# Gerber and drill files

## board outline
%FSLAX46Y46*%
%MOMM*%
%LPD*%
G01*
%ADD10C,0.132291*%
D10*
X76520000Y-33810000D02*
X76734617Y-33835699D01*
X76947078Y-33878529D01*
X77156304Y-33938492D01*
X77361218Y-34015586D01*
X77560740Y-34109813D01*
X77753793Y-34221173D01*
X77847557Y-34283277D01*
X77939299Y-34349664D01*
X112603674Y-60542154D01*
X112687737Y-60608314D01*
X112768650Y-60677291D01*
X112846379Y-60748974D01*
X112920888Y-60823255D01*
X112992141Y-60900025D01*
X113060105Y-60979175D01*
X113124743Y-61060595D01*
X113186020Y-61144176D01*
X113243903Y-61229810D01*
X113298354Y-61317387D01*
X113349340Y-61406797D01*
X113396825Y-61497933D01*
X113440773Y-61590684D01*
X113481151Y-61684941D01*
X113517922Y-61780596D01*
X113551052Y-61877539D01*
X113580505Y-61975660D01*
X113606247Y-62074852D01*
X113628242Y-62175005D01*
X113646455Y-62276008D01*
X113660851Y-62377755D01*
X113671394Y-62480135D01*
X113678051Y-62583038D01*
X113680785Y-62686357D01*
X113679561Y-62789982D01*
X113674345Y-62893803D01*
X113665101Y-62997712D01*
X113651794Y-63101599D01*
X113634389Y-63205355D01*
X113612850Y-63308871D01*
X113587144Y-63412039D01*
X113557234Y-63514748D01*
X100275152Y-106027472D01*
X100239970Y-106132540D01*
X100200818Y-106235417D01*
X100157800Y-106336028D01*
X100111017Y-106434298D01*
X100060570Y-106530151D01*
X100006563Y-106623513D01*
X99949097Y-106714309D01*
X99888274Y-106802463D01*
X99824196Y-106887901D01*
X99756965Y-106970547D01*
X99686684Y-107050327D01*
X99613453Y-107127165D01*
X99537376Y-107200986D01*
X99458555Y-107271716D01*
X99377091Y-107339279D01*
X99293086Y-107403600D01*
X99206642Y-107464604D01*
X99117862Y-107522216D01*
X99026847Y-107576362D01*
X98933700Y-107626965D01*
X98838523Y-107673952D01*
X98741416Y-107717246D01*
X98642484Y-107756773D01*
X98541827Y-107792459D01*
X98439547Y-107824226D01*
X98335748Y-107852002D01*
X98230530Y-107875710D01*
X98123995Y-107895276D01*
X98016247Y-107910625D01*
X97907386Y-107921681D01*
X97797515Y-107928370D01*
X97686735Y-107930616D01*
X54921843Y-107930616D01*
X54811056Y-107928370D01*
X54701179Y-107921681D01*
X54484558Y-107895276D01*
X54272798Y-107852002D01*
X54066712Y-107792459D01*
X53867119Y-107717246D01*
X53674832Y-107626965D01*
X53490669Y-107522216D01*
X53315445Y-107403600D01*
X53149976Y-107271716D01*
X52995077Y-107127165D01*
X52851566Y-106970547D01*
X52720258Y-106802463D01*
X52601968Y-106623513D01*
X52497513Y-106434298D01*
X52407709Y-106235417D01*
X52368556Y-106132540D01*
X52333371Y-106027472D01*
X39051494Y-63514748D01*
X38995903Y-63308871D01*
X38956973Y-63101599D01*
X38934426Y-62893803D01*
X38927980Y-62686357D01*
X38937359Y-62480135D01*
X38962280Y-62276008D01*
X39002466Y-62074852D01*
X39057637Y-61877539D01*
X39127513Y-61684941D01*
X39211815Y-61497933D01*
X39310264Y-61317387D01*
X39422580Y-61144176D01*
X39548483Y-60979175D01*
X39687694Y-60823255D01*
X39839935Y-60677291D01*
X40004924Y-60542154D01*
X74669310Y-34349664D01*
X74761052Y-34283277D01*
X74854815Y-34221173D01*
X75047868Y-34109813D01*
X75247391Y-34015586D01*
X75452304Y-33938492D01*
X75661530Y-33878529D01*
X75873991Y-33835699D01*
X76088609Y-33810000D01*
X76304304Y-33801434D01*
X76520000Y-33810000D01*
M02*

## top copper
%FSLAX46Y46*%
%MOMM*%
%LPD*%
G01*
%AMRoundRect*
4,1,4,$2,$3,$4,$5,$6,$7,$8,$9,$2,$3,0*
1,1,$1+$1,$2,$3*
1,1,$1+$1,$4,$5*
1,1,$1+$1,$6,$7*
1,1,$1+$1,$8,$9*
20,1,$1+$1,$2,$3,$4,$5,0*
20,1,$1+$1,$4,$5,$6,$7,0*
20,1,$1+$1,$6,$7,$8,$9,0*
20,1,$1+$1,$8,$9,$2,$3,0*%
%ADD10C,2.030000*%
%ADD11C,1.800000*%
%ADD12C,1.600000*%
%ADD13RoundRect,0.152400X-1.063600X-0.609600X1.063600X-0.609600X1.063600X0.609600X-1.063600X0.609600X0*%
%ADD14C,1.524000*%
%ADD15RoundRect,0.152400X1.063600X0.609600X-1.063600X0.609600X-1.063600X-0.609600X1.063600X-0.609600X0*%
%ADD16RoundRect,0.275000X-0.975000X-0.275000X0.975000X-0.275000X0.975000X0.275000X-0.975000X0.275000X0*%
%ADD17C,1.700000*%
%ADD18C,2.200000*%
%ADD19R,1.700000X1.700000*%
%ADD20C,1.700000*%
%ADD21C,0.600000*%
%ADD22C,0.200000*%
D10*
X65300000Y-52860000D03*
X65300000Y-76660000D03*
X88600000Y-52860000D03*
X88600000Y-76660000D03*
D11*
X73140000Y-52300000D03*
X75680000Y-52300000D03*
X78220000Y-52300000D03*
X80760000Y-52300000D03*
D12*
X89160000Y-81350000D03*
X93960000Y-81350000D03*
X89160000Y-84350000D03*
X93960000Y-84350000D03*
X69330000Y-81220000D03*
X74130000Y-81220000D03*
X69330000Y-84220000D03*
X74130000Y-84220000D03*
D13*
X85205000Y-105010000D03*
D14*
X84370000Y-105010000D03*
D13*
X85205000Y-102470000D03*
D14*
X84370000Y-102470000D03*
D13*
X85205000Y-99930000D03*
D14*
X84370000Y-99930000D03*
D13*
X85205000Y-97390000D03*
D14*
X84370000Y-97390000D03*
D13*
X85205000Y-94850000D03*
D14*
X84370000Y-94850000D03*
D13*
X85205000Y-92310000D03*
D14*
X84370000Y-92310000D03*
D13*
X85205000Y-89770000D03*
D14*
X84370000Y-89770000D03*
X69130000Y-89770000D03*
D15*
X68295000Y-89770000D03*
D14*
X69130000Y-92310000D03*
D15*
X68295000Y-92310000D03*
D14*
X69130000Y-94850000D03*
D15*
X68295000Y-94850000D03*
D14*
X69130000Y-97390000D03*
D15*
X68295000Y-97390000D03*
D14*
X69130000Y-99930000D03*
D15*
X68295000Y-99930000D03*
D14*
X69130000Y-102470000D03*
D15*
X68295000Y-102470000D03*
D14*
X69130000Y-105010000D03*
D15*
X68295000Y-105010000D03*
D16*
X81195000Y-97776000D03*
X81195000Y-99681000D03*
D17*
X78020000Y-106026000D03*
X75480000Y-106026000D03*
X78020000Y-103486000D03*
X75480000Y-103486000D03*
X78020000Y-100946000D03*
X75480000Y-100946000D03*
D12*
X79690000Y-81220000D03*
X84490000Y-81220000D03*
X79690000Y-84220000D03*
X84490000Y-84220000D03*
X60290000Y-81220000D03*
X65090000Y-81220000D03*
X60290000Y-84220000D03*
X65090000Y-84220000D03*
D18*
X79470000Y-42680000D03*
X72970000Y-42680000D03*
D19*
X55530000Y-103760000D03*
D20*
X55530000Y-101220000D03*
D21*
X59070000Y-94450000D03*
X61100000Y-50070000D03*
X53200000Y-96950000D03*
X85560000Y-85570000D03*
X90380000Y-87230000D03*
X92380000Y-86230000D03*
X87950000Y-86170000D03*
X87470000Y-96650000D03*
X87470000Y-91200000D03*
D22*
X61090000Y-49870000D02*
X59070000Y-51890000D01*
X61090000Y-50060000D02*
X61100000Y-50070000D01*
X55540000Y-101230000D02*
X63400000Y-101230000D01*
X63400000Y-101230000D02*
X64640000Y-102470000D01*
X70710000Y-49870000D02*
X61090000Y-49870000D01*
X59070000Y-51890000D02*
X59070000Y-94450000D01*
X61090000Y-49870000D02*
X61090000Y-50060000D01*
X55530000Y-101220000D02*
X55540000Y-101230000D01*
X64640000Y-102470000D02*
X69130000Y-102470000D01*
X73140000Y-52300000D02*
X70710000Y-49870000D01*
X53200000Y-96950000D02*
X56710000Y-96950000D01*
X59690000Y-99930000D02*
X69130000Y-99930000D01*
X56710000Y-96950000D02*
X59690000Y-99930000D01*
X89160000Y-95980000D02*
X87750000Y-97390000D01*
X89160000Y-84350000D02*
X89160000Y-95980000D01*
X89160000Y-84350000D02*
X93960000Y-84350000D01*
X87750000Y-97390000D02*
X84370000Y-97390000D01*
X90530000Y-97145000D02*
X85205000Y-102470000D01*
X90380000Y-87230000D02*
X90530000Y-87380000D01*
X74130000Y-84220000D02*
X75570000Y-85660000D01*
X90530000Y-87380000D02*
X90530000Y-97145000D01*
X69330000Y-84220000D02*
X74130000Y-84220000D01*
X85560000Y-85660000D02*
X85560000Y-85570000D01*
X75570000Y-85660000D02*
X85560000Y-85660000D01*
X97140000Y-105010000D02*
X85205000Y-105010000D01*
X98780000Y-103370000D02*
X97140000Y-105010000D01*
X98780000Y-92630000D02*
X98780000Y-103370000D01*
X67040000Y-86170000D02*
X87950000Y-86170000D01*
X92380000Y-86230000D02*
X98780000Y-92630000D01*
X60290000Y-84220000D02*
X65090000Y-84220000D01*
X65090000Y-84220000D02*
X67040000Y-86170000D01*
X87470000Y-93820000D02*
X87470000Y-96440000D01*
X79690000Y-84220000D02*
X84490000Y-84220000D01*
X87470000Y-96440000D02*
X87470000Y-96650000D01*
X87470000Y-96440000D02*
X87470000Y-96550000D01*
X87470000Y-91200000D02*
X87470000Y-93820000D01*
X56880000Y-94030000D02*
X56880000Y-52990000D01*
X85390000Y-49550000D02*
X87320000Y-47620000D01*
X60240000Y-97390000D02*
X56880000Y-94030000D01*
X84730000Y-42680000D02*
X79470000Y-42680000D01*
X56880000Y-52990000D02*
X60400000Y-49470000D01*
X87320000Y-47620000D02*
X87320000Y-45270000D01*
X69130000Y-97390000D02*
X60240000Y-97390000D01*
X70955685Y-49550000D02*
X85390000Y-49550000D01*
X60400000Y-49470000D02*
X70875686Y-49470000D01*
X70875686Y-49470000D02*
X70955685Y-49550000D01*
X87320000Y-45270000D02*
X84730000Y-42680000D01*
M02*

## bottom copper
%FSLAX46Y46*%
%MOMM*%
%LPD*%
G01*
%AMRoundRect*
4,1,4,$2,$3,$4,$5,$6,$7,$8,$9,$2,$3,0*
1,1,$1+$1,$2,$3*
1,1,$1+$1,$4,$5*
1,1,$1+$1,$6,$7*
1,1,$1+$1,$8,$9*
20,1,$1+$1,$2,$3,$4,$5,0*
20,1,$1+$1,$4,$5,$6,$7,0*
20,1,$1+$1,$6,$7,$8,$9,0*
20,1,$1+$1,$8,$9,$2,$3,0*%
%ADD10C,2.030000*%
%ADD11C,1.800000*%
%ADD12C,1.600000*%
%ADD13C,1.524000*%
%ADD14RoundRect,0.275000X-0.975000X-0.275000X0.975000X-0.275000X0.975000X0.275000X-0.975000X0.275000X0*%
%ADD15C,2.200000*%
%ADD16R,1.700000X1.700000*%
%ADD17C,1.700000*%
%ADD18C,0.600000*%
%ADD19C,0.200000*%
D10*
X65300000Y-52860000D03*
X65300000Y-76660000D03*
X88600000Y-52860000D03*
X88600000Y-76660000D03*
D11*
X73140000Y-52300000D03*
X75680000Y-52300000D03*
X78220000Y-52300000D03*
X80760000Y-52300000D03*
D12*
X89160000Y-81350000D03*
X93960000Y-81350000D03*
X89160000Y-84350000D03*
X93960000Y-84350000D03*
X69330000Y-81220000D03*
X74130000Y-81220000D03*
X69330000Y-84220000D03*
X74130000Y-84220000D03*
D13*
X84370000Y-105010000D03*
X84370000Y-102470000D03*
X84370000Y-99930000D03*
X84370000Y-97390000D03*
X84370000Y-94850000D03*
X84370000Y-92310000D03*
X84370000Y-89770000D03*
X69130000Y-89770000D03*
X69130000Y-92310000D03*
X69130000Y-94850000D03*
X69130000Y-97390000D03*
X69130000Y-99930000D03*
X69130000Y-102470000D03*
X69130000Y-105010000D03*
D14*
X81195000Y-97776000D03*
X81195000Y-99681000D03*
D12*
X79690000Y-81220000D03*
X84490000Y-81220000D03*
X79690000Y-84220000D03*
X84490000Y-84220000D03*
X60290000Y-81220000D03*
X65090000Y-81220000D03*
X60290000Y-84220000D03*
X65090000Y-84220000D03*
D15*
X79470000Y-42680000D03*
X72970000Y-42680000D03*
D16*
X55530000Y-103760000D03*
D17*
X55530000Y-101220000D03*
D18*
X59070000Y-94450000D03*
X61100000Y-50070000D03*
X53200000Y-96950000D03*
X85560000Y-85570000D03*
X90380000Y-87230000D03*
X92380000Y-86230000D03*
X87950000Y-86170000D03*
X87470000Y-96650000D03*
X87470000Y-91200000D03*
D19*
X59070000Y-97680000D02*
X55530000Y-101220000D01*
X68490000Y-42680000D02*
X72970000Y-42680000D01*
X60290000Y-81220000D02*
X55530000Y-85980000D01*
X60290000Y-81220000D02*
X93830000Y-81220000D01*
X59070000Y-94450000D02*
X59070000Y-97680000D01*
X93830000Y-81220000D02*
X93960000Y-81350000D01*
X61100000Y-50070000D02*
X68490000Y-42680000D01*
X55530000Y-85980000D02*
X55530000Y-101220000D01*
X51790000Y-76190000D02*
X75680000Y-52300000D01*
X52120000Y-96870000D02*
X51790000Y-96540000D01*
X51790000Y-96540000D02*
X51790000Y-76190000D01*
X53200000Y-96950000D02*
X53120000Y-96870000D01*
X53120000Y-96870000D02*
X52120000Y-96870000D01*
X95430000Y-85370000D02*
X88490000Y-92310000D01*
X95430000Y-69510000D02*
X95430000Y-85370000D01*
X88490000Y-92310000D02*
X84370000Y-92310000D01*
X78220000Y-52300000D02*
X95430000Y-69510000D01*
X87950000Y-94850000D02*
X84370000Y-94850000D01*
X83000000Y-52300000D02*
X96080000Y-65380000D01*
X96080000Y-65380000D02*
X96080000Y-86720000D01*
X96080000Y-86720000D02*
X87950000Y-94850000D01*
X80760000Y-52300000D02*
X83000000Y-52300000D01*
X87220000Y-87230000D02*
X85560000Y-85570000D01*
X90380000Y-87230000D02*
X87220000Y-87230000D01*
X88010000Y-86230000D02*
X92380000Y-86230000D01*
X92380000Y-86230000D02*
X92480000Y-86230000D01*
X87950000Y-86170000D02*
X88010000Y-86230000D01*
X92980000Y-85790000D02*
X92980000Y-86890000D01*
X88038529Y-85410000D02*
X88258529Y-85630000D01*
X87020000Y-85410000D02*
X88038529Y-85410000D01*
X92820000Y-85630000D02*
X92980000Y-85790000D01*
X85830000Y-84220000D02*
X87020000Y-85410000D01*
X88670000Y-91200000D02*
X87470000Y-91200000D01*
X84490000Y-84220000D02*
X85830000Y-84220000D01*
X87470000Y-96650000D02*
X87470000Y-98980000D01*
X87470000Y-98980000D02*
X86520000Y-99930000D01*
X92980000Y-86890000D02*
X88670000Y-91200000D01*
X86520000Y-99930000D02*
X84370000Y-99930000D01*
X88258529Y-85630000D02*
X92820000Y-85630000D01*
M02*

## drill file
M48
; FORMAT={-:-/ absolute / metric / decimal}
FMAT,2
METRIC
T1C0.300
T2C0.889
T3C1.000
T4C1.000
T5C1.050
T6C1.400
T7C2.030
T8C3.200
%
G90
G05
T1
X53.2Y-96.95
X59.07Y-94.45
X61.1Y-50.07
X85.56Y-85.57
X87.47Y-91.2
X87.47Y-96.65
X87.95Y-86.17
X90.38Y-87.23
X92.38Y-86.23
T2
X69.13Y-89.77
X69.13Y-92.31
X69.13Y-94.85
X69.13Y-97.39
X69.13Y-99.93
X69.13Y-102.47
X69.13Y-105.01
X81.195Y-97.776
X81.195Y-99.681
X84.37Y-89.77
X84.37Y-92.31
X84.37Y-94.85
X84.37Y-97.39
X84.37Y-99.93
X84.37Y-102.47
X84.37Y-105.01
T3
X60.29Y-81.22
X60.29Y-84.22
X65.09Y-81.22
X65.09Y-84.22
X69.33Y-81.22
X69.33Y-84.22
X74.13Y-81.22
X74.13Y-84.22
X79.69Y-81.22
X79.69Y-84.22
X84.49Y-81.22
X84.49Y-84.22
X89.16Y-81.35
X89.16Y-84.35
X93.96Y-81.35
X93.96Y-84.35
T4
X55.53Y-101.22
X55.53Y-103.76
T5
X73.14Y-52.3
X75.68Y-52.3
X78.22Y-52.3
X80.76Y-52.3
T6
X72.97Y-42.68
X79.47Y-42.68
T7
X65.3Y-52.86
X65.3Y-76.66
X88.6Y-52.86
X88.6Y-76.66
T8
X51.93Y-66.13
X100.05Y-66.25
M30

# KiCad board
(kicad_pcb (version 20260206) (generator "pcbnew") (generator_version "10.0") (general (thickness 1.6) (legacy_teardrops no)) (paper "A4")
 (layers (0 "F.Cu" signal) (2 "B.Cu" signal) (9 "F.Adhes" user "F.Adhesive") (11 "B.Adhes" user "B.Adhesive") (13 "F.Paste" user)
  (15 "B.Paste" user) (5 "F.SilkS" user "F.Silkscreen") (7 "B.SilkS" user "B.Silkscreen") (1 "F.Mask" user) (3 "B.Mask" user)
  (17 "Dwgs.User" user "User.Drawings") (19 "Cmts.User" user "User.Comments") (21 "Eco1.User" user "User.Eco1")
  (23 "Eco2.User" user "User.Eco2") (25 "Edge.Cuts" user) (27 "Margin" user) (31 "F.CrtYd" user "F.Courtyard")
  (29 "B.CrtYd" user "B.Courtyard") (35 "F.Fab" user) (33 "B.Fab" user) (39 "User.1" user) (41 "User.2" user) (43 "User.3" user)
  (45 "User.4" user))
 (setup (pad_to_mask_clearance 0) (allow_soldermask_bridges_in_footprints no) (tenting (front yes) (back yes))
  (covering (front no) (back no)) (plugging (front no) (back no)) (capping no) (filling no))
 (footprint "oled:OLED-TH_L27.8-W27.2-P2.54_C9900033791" (layer "F.Cu") (at 76.95 52.3)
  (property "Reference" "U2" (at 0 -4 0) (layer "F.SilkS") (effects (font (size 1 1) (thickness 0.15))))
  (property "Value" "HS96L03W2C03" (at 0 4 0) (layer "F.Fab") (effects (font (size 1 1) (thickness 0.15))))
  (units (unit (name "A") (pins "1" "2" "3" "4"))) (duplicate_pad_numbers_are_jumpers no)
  (pad "" thru_hole circle (at -11.65 0.56) (size 2.03 2.03) (drill 2.03) (layers "*.Cu" "*.Mask") (remove_unused_layers no))
  (pad "" thru_hole circle (at -11.65 24.36) (size 2.03 2.03) (drill 2.03) (layers "*.Cu" "*.Mask") (remove_unused_layers no))
  (pad "" thru_hole circle (at 11.65 0.56) (size 2.03 2.03) (drill 2.03) (layers "*.Cu" "*.Mask") (remove_unused_layers no))
  (pad "" thru_hole circle (at 11.65 24.36) (size 2.03 2.03) (drill 2.03) (layers "*.Cu" "*.Mask") (remove_unused_layers no))
  (pad "1" thru_hole circle (at -3.81 0) (size 1.8 1.8) (drill 1.049986) (layers "*.Cu" "*.Mask") (remove_unused_layers no) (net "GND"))
  (pad "2" thru_hole circle (at -1.27 0) (size 1.8 1.8) (drill 1.049986) (layers "*.Cu" "*.Mask") (remove_unused_layers no) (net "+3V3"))
  (pad "3" thru_hole circle (at 1.27 0) (size 1.8 1.8) (drill 1.049986) (layers "*.Cu" "*.Mask") (remove_unused_layers no)
   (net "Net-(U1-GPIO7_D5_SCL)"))
  (pad "4" thru_hole circle (at 3.81 0) (size 1.8 1.8) (drill 1.049986) (layers "*.Cu" "*.Mask") (remove_unused_layers no)
   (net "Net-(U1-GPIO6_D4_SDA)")))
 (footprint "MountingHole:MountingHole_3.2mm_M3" (layer "F.Cu") (at 100.05 66.25)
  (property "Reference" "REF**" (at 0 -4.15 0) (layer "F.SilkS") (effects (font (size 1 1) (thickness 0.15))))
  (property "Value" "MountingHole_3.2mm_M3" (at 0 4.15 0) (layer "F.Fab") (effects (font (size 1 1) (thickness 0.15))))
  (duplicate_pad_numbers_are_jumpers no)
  (pad "" np_thru_hole circle (at 0 0) (size 3.2 3.2) (drill 3.2) (layers "*.Cu" "*.Mask")))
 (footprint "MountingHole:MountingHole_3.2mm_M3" (layer "F.Cu") (at 51.93 66.13)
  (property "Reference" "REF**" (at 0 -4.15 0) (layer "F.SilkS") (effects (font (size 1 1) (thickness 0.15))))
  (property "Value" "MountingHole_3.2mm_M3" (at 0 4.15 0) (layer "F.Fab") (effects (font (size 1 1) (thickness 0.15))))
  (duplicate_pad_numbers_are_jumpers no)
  (pad "" np_thru_hole circle (at 0 0) (size 3.2 3.2) (drill 3.2) (layers "*.Cu" "*.Mask")))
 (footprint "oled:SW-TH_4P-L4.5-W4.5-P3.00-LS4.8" (layer "F.Cu") (at 91.56 82.85)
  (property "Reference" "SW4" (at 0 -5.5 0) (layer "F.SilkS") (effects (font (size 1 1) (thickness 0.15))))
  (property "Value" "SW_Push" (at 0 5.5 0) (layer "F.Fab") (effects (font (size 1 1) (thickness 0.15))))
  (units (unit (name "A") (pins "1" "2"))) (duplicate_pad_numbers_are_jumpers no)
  (pad "1" thru_hole circle (at -2.4 -1.5) (size 1.6 1.6) (drill 0.999998) (layers "*.Cu" "*.Mask") (remove_unused_layers no) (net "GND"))
  (pad "1" thru_hole circle (at 2.4 -1.5) (size 1.6 1.6) (drill 0.999998) (layers "*.Cu" "*.Mask") (remove_unused_layers no) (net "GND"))
  (pad "2" thru_hole circle (at -2.4 1.5) (size 1.6 1.6) (drill 0.999998) (layers "*.Cu" "*.Mask") (remove_unused_layers no)
   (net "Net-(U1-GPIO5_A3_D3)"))
  (pad "2" thru_hole circle (at 2.4 1.5) (size 1.6 1.6) (drill 0.999998) (layers "*.Cu" "*.Mask") (remove_unused_layers no)
   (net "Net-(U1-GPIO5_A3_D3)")))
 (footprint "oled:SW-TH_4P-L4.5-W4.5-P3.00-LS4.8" (layer "F.Cu") (at 71.73 82.72)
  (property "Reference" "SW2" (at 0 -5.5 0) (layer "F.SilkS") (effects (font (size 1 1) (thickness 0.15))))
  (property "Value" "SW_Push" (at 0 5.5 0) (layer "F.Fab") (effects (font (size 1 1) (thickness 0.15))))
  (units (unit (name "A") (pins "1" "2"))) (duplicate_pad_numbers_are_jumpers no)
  (pad "1" thru_hole circle (at -2.4 -1.5) (size 1.6 1.6) (drill 0.999998) (layers "*.Cu" "*.Mask") (remove_unused_layers no) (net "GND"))
  (pad "1" thru_hole circle (at 2.4 -1.5) (size 1.6 1.6) (drill 0.999998) (layers "*.Cu" "*.Mask") (remove_unused_layers no) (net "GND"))
  (pad "2" thru_hole circle (at -2.4 1.5) (size 1.6 1.6) (drill 0.999998) (layers "*.Cu" "*.Mask") (remove_unused_layers no)
   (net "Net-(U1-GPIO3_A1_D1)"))
  (pad "2" thru_hole circle (at 2.4 1.5) (size 1.6 1.6) (drill 0.999998) (layers "*.Cu" "*.Mask") (remove_unused_layers no)
   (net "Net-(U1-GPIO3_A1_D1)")))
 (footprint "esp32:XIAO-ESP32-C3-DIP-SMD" (layer "F.Cu") (at 76.75 97.39 -90)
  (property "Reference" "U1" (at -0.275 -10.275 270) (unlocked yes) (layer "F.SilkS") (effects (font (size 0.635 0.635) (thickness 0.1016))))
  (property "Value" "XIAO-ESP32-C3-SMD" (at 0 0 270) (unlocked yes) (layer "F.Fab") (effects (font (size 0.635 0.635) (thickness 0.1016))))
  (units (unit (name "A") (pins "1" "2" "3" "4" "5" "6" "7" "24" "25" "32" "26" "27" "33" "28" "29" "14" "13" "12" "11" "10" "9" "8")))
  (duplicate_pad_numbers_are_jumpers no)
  (pad "1" smd roundrect (at 7.62 -8.455) (size 2.432 1.524) (layers "F.Cu" "F.Mask") (roundrect_rratio 0.1) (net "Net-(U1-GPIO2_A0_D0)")
   (thermal_bridge_angle 45))
  (pad "1" thru_hole circle (at 7.62 -7.62) (size 1.524 1.524) (drill 0.889) (layers "*.Cu" "*.Mask") (remove_unused_layers no)
   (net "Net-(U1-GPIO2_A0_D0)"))
  (pad "2" smd roundrect (at 5.08 -8.455) (size 2.432 1.524) (layers "F.Cu" "F.Mask") (roundrect_rratio 0.1) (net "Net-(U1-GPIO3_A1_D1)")
   (thermal_bridge_angle 45))
  (pad "2" thru_hole circle (at 5.08 -7.62) (size 1.524 1.524) (drill 0.889) (layers "*.Cu" "*.Mask") (remove_unused_layers no)
   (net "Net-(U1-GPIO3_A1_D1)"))
  (pad "3" smd roundrect (at 2.54 -8.455) (size 2.432 1.524) (layers "F.Cu" "F.Mask") (roundrect_rratio 0.1) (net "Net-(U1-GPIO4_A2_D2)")
   (thermal_bridge_angle 45))
  (pad "3" thru_hole circle (at 2.54 -7.62) (size 1.524 1.524) (drill 0.889) (layers "*.Cu" "*.Mask") (remove_unused_layers no)
   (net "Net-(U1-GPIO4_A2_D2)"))
  (pad "4" smd roundrect (at 0 -8.455) (size 2.432 1.524) (layers "F.Cu" "F.Mask") (roundrect_rratio 0.1) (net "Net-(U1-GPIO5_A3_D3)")
   (thermal_bridge_angle 45))
  (pad "4" thru_hole circle (at 0 -7.62) (size 1.524 1.524) (drill 0.889) (layers "*.Cu" "*.Mask") (remove_unused_layers no)
   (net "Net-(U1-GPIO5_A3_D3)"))
  (pad "5" smd roundrect (at -2.54 -8.455) (size 2.432 1.524) (layers "F.Cu" "F.Mask") (roundrect_rratio 0.1) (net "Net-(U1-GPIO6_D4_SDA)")
   (thermal_bridge_angle 45))
  (pad "5" thru_hole circle (at -2.54 -7.62) (size 1.524 1.524) (drill 0.889) (layers "*.Cu" "*.Mask") (remove_unused_layers no)
   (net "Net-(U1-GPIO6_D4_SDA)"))
  (pad "6" smd roundrect (at -5.08 -8.455) (size 2.432 1.524) (layers "F.Cu" "F.Mask") (roundrect_rratio 0.1) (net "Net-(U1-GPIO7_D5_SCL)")
   (thermal_bridge_angle 45))
  (pad "6" thru_hole circle (at -5.08 -7.62) (size 1.524 1.524) (drill 0.889) (layers "*.Cu" "*.Mask") (remove_unused_layers no)
   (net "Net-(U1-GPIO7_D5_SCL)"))
  (pad "7" smd roundrect (at -7.62 -8.455) (size 2.432 1.524) (layers "F.Cu" "F.Mask") (roundrect_rratio 0.1)
   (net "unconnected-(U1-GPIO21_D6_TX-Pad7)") (thermal_bridge_angle 45))
  (pad "7" thru_hole circle (at -7.62 -7.62) (size 1.524 1.524) (drill 0.889) (layers "*.Cu" "*.Mask") (remove_unused_layers no)
   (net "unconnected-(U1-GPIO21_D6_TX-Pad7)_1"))
  (pad "8" thru_hole circle (at -7.62 7.62 180) (size 1.524 1.524) (drill 0.889) (layers "*.Cu" "*.Mask") (remove_unused_layers no)
   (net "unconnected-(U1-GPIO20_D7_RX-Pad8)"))
  (pad "8" smd roundrect (at -7.62 8.455 180) (size 2.432 1.524) (layers "F.Cu" "F.Mask") (roundrect_rratio 0.1)
   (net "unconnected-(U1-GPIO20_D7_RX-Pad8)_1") (thermal_bridge_angle 45))
  (pad "9" thru_hole circle (at -5.08 7.62 180) (size 1.524 1.524) (drill 0.889) (layers "*.Cu" "*.Mask") (remove_unused_layers no)
   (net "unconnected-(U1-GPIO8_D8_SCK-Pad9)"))
  (pad "9" smd roundrect (at -5.08 8.455 180) (size 2.432 1.524) (layers "F.Cu" "F.Mask") (roundrect_rratio 0.1)
   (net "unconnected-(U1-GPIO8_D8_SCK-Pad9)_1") (thermal_bridge_angle 45))
  (pad "10" thru_hole circle (at -2.54 7.62 180) (size 1.524 1.524) (drill 0.889) (layers "*.Cu" "*.Mask") (remove_unused_layers no)
   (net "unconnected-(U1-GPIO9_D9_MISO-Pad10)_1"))
  (pad "10" smd roundrect (at -2.54 8.455 180) (size 2.432 1.524) (layers "F.Cu" "F.Mask") (roundrect_rratio 0.1)
   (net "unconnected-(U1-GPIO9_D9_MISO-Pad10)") (thermal_bridge_angle 45))
  (pad "11" thru_hole circle (at 0 7.62 180) (size 1.524 1.524) (drill 0.889) (layers "*.Cu" "*.Mask") (remove_unused_layers no)
   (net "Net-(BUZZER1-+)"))
  (pad "11" smd roundrect (at 0 8.455 180) (size 2.432 1.524) (layers "F.Cu" "F.Mask") (roundrect_rratio 0.1) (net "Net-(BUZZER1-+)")
   (thermal_bridge_angle 45))
  (pad "12" thru_hole circle (at 2.54 7.62 180) (size 1.524 1.524) (drill 0.889) (layers "*.Cu" "*.Mask") (remove_unused_layers no)
   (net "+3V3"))
  (pad "12" smd roundrect (at 2.54 8.455 180) (size 2.432 1.524) (layers "F.Cu" "F.Mask") (roundrect_rratio 0.1) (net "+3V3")
   (thermal_bridge_angle 45))
  (pad "13" thru_hole circle (at 5.08 7.62 180) (size 1.524 1.524) (drill 0.889) (layers "*.Cu" "*.Mask") (remove_unused_layers no)
   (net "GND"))
  (pad "13" smd roundrect (at 5.08 8.455 180) (size 2.432 1.524) (layers "F.Cu" "F.Mask") (roundrect_rratio 0.1) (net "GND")
   (thermal_bridge_angle 45))
  (pad "14" thru_hole circle (at 7.62 7.62 180) (size 1.524 1.524) (drill 0.889) (layers "*.Cu" "*.Mask") (remove_unused_layers no)
   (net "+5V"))
  (pad "14" smd roundrect (at 7.62 8.455 180) (size 2.432 1.524) (layers "F.Cu" "F.Mask") (roundrect_rratio 0.1) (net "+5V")
   (thermal_bridge_angle 45))
  (pad "15" thru_hole roundrect (at 0.386 -4.445) (size 2.5 1.1) (drill 0.889) (layers "*.Cu" "*.Mask") (remove_unused_layers no)
   (roundrect_rratio 0.25) (thermal_bridge_angle 45))
  (pad "16" thru_hole roundrect (at 2.291 -4.445) (size 2.5 1.1) (drill 0.889) (layers "*.Cu" "*.Mask") (remove_unused_layers no)
   (roundrect_rratio 0.25) (thermal_bridge_angle 45))
  (pad "17" smd circle (at 8.636 -1.27 180) (size 1.7 1.7) (layers "F.Cu" "F.Mask" "F.Paste"))
  (pad "18" smd circle (at 8.636 1.27 180) (size 1.7 1.7) (layers "F.Cu" "F.Mask" "F.Paste"))
  (pad "19" smd circle (at 6.096 -1.27 180) (size 1.7 1.7) (layers "F.Cu" "F.Mask" "F.Paste"))
  (pad "20" smd circle (at 6.096 1.27 180) (size 1.7 1.7) (layers "F.Cu" "F.Mask" "F.Paste"))
  (pad "21" smd circle (at 3.556 -1.27 180) (size 1.7 1.7) (layers "F.Cu" "F.Mask" "F.Paste"))
  (pad "22" smd circle (at 3.556 1.27 180) (size 1.7 1.7) (layers "F.Cu" "F.Mask" "F.Paste")))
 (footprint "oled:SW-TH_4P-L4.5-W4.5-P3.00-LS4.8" (layer "F.Cu") (at 82.09 82.72)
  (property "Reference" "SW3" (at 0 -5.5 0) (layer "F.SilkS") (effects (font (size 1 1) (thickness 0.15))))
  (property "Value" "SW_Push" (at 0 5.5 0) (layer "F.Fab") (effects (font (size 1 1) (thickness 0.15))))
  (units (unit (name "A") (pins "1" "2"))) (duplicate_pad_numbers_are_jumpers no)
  (pad "1" thru_hole circle (at -2.4 -1.5) (size 1.6 1.6) (drill 0.999998) (layers "*.Cu" "*.Mask") (remove_unused_layers no) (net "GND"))
  (pad "1" thru_hole circle (at 2.4 -1.5) (size 1.6 1.6) (drill 0.999998) (layers "*.Cu" "*.Mask") (remove_unused_layers no) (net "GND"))
  (pad "2" thru_hole circle (at -2.4 1.5) (size 1.6 1.6) (drill 0.999998) (layers "*.Cu" "*.Mask") (remove_unused_layers no)
   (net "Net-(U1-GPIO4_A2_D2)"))
  (pad "2" thru_hole circle (at 2.4 1.5) (size 1.6 1.6) (drill 0.999998) (layers "*.Cu" "*.Mask") (remove_unused_layers no)
   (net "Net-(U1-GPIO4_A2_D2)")))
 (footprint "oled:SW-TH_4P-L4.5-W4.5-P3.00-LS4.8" (layer "F.Cu") (at 62.69 82.72)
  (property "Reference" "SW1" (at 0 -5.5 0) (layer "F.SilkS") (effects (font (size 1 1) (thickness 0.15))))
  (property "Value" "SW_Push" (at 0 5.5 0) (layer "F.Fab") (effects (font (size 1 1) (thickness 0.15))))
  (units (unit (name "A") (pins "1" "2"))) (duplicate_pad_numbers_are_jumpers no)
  (pad "1" thru_hole circle (at -2.4 -1.5) (size 1.6 1.6) (drill 0.999998) (layers "*.Cu" "*.Mask") (remove_unused_layers no) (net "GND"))
  (pad "1" thru_hole circle (at 2.4 -1.5) (size 1.6 1.6) (drill 0.999998) (layers "*.Cu" "*.Mask") (remove_unused_layers no) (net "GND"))
  (pad "2" thru_hole circle (at -2.4 1.5) (size 1.6 1.6) (drill 0.999998) (layers "*.Cu" "*.Mask") (remove_unused_layers no)
   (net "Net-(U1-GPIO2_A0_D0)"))
  (pad "2" thru_hole circle (at 2.4 1.5) (size 1.6 1.6) (drill 0.999998) (layers "*.Cu" "*.Mask") (remove_unused_layers no)
   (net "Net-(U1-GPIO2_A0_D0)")))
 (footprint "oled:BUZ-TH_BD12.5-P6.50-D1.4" (layer "B.Cu") (at 76.22 42.68 180)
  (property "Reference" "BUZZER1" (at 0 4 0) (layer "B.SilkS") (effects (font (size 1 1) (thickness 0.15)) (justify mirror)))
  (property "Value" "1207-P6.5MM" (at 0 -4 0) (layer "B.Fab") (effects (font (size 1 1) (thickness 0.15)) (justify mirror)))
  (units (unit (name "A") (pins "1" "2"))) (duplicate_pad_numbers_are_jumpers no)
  (pad "1" thru_hole circle (at -3.25 0 180) (size 2.2 2.2) (drill 1.399998) (layers "*.Cu" "*.Mask") (remove_unused_layers no)
   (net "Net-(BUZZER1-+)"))
  (pad "2" thru_hole circle (at 3.25 0 180) (size 2.2 2.2) (drill 1.399998) (layers "*.Cu" "*.Mask") (remove_unused_layers no) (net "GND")))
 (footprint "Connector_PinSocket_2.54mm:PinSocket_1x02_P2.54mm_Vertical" (layer "B.Cu") (at 55.53 103.76)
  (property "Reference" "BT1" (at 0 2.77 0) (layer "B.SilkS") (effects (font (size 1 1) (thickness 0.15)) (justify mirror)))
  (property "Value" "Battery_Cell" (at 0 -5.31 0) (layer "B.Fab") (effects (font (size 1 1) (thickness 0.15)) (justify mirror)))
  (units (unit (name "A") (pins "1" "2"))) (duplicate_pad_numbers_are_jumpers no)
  (pad "1" thru_hole rect (at 0 0) (size 1.7 1.7) (drill 1) (layers "*.Cu" "*.Mask") (remove_unused_layers no) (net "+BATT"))
  (pad "2" thru_hole circle (at 0 -2.54) (size 1.7 1.7) (drill 1) (layers "*.Cu" "*.Mask") (remove_unused_layers no) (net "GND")))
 (gr_poly
  (pts (xy 76.52 33.81) (xy 76.734617 33.835699) (xy 76.947078 33.878529) (xy 77.156304 33.938492) (xy 77.361218 34.015586)
   (xy 77.56074 34.109813) (xy 77.753793 34.221173) (xy 77.847557 34.283277) (xy 77.939299 34.349664) (xy 112.603674 60.542154)
   (xy 112.687737 60.608314) (xy 112.76865 60.677291) (xy 112.846379 60.748974) (xy 112.920888 60.823255) (xy 112.992141 60.900025)
   (xy 113.060105 60.979175) (xy 113.124743 61.060595) (xy 113.18602 61.144176) (xy 113.243903 61.22981) (xy 113.298354 61.317387)
   (xy 113.34934 61.406797) (xy 113.396825 61.497933) (xy 113.440773 61.590684) (xy 113.481151 61.684941) (xy 113.517922 61.780596)
   (xy 113.551052 61.877539) (xy 113.580505 61.97566) (xy 113.606247 62.074852) (xy 113.628242 62.175005) (xy 113.646455 62.276008)
   (xy 113.660851 62.377755) (xy 113.671394 62.480135) (xy 113.678051 62.583038) (xy 113.680785 62.686357) (xy 113.679561 62.789982)
   (xy 113.674345 62.893803) (xy 113.665101 62.997712) (xy 113.651794 63.101599) (xy 113.634389 63.205355) (xy 113.61285 63.308871)
   (xy 113.587144 63.412039) (xy 113.557234 63.514748) (xy 100.275152 106.027472) (xy 100.23997 106.13254) (xy 100.200818 106.235417)
   (xy 100.1578 106.336028) (xy 100.111017 106.434298) (xy 100.06057 106.530151) (xy 100.006563 106.623513) (xy 99.949097 106.714309)
   (xy 99.888274 106.802463) (xy 99.824196 106.887901) (xy 99.756965 106.970547) (xy 99.686684 107.050327) (xy 99.613453 107.127165)
   (xy 99.537376 107.200986) (xy 99.458555 107.271716) (xy 99.377091 107.339279) (xy 99.293086 107.4036) (xy 99.206642 107.464604)
   (xy 99.117862 107.522216) (xy 99.026847 107.576362) (xy 98.9337 107.626965) (xy 98.838523 107.673952) (xy 98.741416 107.717246)
   (xy 98.642484 107.756773) (xy 98.541827 107.792459) (xy 98.439547 107.824226) (xy 98.335748 107.852002) (xy 98.23053 107.87571)
   (xy 98.123995 107.895276) (xy 98.016247 107.910625) (xy 97.907386 107.921681) (xy 97.797515 107.92837) (xy 97.686735 107.930616)
   (xy 54.921843 107.930616) (xy 54.811056 107.92837) (xy 54.701179 107.921681) (xy 54.484558 107.895276) (xy 54.272798 107.852002)
   (xy 54.066712 107.792459) (xy 53.867119 107.717246) (xy 53.674832 107.626965) (xy 53.490669 107.522216) (xy 53.315445 107.4036)
   (xy 53.149976 107.271716) (xy 52.995077 107.127165) (xy 52.851566 106.970547) (xy 52.720258 106.802463) (xy 52.601968 106.623513)
   (xy 52.497513 106.434298) (xy 52.407709 106.235417) (xy 52.368556 106.13254) (xy 52.333371 106.027472) (xy 39.051494 63.514748)
   (xy 38.995903 63.308871) (xy 38.956973 63.101599) (xy 38.934426 62.893803) (xy 38.92798 62.686357) (xy 38.937359 62.480135)
   (xy 38.96228 62.276008) (xy 39.002466 62.074852) (xy 39.057637 61.877539) (xy 39.127513 61.684941) (xy 39.211815 61.497933)
   (xy 39.310264 61.317387) (xy 39.42258 61.144176) (xy 39.548483 60.979175) (xy 39.687694 60.823255) (xy 39.839935 60.677291)
   (xy 40.004924 60.542154) (xy 74.66931 34.349664) (xy 74.761052 34.283277) (xy 74.854815 34.221173) (xy 75.047868 34.109813)
   (xy 75.247391 34.015586) (xy 75.452304 33.938492) (xy 75.66153 33.878529) (xy 75.873991 33.835699) (xy 76.088609 33.81)
   (xy 76.304304 33.801434))
  (stroke (width 0.132291) (type solid)) (fill no) (layer "Edge.Cuts"))
 (segment (start 61.09 49.87) (end 59.07 51.89) (width 0.2) (layer "F.Cu") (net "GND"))
 (segment (start 61.09 50.06) (end 61.1 50.07) (width 0.2) (layer "F.Cu") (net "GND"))
 (segment (start 55.54 101.23) (end 63.4 101.23) (width 0.2) (layer "F.Cu") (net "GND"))
 (segment (start 63.4 101.23) (end 64.64 102.47) (width 0.2) (layer "F.Cu") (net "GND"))
 (segment (start 70.71 49.87) (end 61.09 49.87) (width 0.2) (layer "F.Cu") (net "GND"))
 (segment (start 59.07 51.89) (end 59.07 94.45) (width 0.2) (layer "F.Cu") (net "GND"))
 (segment (start 61.09 49.87) (end 61.09 50.06) (width 0.2) (layer "F.Cu") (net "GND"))
 (segment (start 55.53 101.22) (end 55.54 101.23) (width 0.2) (layer "F.Cu") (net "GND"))
 (segment (start 64.64 102.47) (end 69.13 102.47) (width 0.2) (layer "F.Cu") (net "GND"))
 (segment (start 73.14 52.3) (end 70.71 49.87) (width 0.2) (layer "F.Cu") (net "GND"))
 (via (at 59.07 94.45) (size 0.6) (drill 0.3) (layers "F.Cu" "B.Cu") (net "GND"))
 (via (at 61.1 50.07) (size 0.6) (drill 0.3) (layers "F.Cu" "B.Cu") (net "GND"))
 (segment (start 59.07 97.68) (end 55.53 101.22) (width 0.2) (layer "B.Cu") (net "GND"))
 (segment (start 68.49 42.68) (end 72.97 42.68) (width 0.2) (layer "B.Cu") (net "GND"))
 (segment (start 60.29 81.22) (end 55.53 85.98) (width 0.2) (layer "B.Cu") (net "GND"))
 (segment (start 60.29 81.22) (end 93.83 81.22) (width 0.2) (layer "B.Cu") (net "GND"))
 (segment (start 59.07 94.45) (end 59.07 97.68) (width 0.2) (layer "B.Cu") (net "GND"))
 (segment (start 93.83 81.22) (end 93.96 81.35) (width 0.2) (layer "B.Cu") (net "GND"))
 (segment (start 61.1 50.07) (end 68.49 42.68) (width 0.2) (layer "B.Cu") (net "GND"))
 (segment (start 55.53 85.98) (end 55.53 101.22) (width 0.2) (layer "B.Cu") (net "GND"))
 (segment (start 53.2 96.95) (end 56.71 96.95) (width 0.2) (layer "F.Cu") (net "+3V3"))
 (segment (start 59.69 99.93) (end 69.13 99.93) (width 0.2) (layer "F.Cu") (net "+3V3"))
 (segment (start 56.71 96.95) (end 59.69 99.93) (width 0.2) (layer "F.Cu") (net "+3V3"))
 (via (at 53.2 96.95) (size 0.6) (drill 0.3) (layers "F.Cu" "B.Cu") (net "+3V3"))
 (segment (start 51.79 76.19) (end 75.68 52.3) (width 0.2) (layer "B.Cu") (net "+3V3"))
 (segment (start 52.12 96.87) (end 51.79 96.54) (width 0.2) (layer "B.Cu") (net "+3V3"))
 (segment (start 51.79 96.54) (end 51.79 76.19) (width 0.2) (layer "B.Cu") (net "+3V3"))
 (segment (start 53.2 96.95) (end 53.12 96.87) (width 0.2) (layer "B.Cu") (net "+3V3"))
 (segment (start 53.12 96.87) (end 52.12 96.87) (width 0.2) (layer "B.Cu") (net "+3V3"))
 (segment (start 95.43 85.37) (end 88.49 92.31) (width 0.2) (layer "B.Cu") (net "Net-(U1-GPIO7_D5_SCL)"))
 (segment (start 95.43 69.51) (end 95.43 85.37) (width 0.2) (layer "B.Cu") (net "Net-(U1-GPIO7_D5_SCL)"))
 (segment (start 88.49 92.31) (end 84.37 92.31) (width 0.2) (layer "B.Cu") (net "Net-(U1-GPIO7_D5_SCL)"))
 (segment (start 78.22 52.3) (end 95.43 69.51) (width 0.2) (layer "B.Cu") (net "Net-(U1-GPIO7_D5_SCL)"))
 (segment (start 87.95 94.85) (end 84.37 94.85) (width 0.2) (layer "B.Cu") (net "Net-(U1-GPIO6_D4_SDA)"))
 (segment (start 83 52.3) (end 96.08 65.38) (width 0.2) (layer "B.Cu") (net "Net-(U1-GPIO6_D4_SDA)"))
 (segment (start 96.08 65.38) (end 96.08 86.72) (width 0.2) (layer "B.Cu") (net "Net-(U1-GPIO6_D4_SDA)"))
 (segment (start 96.08 86.72) (end 87.95 94.85) (width 0.2) (layer "B.Cu") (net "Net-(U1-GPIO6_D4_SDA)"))
 (segment (start 80.76 52.3) (end 83 52.3) (width 0.2) (layer "B.Cu") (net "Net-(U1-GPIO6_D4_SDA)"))
 (segment (start 89.16 95.98) (end 87.75 97.39) (width 0.2) (layer "F.Cu") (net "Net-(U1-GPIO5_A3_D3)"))
 (segment (start 89.16 84.35) (end 89.16 95.98) (width 0.2) (layer "F.Cu") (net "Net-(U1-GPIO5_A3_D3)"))
 (segment (start 89.16 84.35) (end 93.96 84.35) (width 0.2) (layer "F.Cu") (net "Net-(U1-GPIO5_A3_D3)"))
 (segment (start 87.75 97.39) (end 84.37 97.39) (width 0.2) (layer "F.Cu") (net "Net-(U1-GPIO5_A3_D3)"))
 (segment (start 90.53 97.145) (end 85.205 102.47) (width 0.2) (layer "F.Cu") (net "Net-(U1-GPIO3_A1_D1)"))
 (segment (start 90.38 87.23) (end 90.53 87.38) (width 0.2) (layer "F.Cu") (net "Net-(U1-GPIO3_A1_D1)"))
 (segment (start 74.13 84.22) (end 75.57 85.66) (width 0.2) (layer "F.Cu") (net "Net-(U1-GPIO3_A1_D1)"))
 (segment (start 90.53 87.38) (end 90.53 97.145) (width 0.2) (layer "F.Cu") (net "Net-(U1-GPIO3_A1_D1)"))
 (segment (start 69.33 84.22) (end 74.13 84.22) (width 0.2) (layer "F.Cu") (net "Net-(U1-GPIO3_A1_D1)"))
 (segment (start 85.56 85.66) (end 85.56 85.57) (width 0.2) (layer "F.Cu") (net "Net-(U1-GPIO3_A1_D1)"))
 (segment (start 75.57 85.66) (end 85.56 85.66) (width 0.2) (layer "F.Cu") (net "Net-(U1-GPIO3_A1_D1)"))
 (via (at 85.56 85.57) (size 0.6) (drill 0.3) (layers "F.Cu" "B.Cu") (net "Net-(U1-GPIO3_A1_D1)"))
 (via (at 90.38 87.23) (size 0.6) (drill 0.3) (layers "F.Cu" "B.Cu") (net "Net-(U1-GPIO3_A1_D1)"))
 (segment (start 87.22 87.23) (end 85.56 85.57) (width 0.2) (layer "B.Cu") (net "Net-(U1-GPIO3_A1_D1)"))
 (segment (start 90.38 87.23) (end 87.22 87.23) (width 0.2) (layer "B.Cu") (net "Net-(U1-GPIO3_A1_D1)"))
 (segment (start 97.14 105.01) (end 85.205 105.01) (width 0.2) (layer "F.Cu") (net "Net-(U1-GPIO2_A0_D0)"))
 (segment (start 98.78 103.37) (end 97.14 105.01) (width 0.2) (layer "F.Cu") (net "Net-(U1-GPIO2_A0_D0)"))
 (segment (start 98.78 92.63) (end 98.78 103.37) (width 0.2) (layer "F.Cu") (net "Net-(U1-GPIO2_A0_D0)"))
 (segment (start 67.04 86.17) (end 87.95 86.17) (width 0.2) (layer "F.Cu") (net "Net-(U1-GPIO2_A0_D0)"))
 (segment (start 92.38 86.23) (end 98.78 92.63) (width 0.2) (layer "F.Cu") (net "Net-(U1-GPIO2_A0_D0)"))
 (segment (start 60.29 84.22) (end 65.09 84.22) (width 0.2) (layer "F.Cu") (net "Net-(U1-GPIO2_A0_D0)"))
 (segment (start 65.09 84.22) (end 67.04 86.17) (width 0.2) (layer "F.Cu") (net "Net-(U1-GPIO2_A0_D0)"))
 (via (at 92.38 86.23) (size 0.6) (drill 0.3) (layers "F.Cu" "B.Cu") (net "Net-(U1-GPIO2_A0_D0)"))
 (via (at 87.95 86.17) (size 0.6) (drill 0.3) (layers "F.Cu" "B.Cu") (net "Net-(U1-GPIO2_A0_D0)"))
 (segment (start 88.01 86.23) (end 92.38 86.23) (width 0.2) (layer "B.Cu") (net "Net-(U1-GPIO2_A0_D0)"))
 (segment (start 92.38 86.23) (end 92.48 86.23) (width 0.2) (layer "B.Cu") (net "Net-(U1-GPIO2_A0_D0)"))
 (segment (start 87.95 86.17) (end 88.01 86.23) (width 0.2) (layer "B.Cu") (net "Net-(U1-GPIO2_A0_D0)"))
 (segment (start 87.47 93.82) (end 87.47 96.44) (width 0.2) (layer "F.Cu") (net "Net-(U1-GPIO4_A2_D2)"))
 (segment (start 79.69 84.22) (end 84.49 84.22) (width 0.2) (layer "F.Cu") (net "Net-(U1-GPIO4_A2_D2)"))
 (segment (start 87.47 96.44) (end 87.47 96.65) (width 0.2) (layer "F.Cu") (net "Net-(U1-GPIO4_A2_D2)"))
 (segment (start 87.47 96.44) (end 87.47 96.55) (width 0.2) (layer "F.Cu") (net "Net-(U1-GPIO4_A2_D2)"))
 (segment (start 87.47 91.2) (end 87.47 93.82) (width 0.2) (layer "F.Cu") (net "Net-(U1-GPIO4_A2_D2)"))
 (via (at 87.47 96.65) (size 0.6) (drill 0.3) (layers "F.Cu" "B.Cu") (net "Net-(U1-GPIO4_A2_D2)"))
 (via (at 87.47 91.2) (size 0.6) (drill 0.3) (layers "F.Cu" "B.Cu") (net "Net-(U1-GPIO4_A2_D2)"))
 (segment (start 92.98 85.79) (end 92.98 86.89) (width 0.2) (layer "B.Cu") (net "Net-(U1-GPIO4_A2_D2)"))
 (segment (start 88.038529 85.41) (end 88.258529 85.63) (width 0.2) (layer "B.Cu") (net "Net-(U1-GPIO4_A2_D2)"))
 (segment (start 87.02 85.41) (end 88.038529 85.41) (width 0.2) (layer "B.Cu") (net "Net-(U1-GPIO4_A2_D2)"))
 (segment (start 92.82 85.63) (end 92.98 85.79) (width 0.2) (layer "B.Cu") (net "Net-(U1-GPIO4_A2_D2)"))
 (segment (start 85.83 84.22) (end 87.02 85.41) (width 0.2) (layer "B.Cu") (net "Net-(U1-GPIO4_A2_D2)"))
 (segment (start 88.67 91.2) (end 87.47 91.2) (width 0.2) (layer "B.Cu") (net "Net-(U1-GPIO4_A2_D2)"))
 (segment (start 84.49 84.22) (end 85.83 84.22) (width 0.2) (layer "B.Cu") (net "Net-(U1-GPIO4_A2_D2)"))
 (segment (start 87.47 96.65) (end 87.47 98.98) (width 0.2) (layer "B.Cu") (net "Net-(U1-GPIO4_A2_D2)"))
 (segment (start 87.47 98.98) (end 86.52 99.93) (width 0.2) (layer "B.Cu") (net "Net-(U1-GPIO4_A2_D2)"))
 (segment (start 92.98 86.89) (end 88.67 91.2) (width 0.2) (layer "B.Cu") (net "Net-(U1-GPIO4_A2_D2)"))
 (segment (start 86.52 99.93) (end 84.37 99.93) (width 0.2) (layer "B.Cu") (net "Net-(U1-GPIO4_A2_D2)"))
 (segment (start 88.258529 85.63) (end 92.82 85.63) (width 0.2) (layer "B.Cu") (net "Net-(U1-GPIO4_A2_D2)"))
 (segment (start 56.88 94.03) (end 56.88 52.99) (width 0.2) (layer "F.Cu") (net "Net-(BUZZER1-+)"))
 (segment (start 85.39 49.55) (end 87.32 47.62) (width 0.2) (layer "F.Cu") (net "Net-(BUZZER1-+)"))
 (segment (start 60.24 97.39) (end 56.88 94.03) (width 0.2) (layer "F.Cu") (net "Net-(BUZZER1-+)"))
 (segment (start 84.73 42.68) (end 79.47 42.68) (width 0.2) (layer "F.Cu") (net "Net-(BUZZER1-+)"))
 (segment (start 56.88 52.99) (end 60.4 49.47) (width 0.2) (layer "F.Cu") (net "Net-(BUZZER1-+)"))
 (segment (start 87.32 47.62) (end 87.32 45.27) (width 0.2) (layer "F.Cu") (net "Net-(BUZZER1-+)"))
 (segment (start 69.13 97.39) (end 60.24 97.39) (width 0.2) (layer "F.Cu") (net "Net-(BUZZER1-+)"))
 (segment (start 70.955685 49.55) (end 85.39 49.55) (width 0.2) (layer "F.Cu") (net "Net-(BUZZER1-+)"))
 (segment (start 60.4 49.47) (end 70.875686 49.47) (width 0.2) (layer "F.Cu") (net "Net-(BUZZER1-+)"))
 (segment (start 70.875686 49.47) (end 70.955685 49.55) (width 0.2) (layer "F.Cu") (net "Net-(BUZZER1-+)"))
 (segment (start 87.32 45.27) (end 84.73 42.68) (width 0.2) (layer "F.Cu") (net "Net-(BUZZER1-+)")))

